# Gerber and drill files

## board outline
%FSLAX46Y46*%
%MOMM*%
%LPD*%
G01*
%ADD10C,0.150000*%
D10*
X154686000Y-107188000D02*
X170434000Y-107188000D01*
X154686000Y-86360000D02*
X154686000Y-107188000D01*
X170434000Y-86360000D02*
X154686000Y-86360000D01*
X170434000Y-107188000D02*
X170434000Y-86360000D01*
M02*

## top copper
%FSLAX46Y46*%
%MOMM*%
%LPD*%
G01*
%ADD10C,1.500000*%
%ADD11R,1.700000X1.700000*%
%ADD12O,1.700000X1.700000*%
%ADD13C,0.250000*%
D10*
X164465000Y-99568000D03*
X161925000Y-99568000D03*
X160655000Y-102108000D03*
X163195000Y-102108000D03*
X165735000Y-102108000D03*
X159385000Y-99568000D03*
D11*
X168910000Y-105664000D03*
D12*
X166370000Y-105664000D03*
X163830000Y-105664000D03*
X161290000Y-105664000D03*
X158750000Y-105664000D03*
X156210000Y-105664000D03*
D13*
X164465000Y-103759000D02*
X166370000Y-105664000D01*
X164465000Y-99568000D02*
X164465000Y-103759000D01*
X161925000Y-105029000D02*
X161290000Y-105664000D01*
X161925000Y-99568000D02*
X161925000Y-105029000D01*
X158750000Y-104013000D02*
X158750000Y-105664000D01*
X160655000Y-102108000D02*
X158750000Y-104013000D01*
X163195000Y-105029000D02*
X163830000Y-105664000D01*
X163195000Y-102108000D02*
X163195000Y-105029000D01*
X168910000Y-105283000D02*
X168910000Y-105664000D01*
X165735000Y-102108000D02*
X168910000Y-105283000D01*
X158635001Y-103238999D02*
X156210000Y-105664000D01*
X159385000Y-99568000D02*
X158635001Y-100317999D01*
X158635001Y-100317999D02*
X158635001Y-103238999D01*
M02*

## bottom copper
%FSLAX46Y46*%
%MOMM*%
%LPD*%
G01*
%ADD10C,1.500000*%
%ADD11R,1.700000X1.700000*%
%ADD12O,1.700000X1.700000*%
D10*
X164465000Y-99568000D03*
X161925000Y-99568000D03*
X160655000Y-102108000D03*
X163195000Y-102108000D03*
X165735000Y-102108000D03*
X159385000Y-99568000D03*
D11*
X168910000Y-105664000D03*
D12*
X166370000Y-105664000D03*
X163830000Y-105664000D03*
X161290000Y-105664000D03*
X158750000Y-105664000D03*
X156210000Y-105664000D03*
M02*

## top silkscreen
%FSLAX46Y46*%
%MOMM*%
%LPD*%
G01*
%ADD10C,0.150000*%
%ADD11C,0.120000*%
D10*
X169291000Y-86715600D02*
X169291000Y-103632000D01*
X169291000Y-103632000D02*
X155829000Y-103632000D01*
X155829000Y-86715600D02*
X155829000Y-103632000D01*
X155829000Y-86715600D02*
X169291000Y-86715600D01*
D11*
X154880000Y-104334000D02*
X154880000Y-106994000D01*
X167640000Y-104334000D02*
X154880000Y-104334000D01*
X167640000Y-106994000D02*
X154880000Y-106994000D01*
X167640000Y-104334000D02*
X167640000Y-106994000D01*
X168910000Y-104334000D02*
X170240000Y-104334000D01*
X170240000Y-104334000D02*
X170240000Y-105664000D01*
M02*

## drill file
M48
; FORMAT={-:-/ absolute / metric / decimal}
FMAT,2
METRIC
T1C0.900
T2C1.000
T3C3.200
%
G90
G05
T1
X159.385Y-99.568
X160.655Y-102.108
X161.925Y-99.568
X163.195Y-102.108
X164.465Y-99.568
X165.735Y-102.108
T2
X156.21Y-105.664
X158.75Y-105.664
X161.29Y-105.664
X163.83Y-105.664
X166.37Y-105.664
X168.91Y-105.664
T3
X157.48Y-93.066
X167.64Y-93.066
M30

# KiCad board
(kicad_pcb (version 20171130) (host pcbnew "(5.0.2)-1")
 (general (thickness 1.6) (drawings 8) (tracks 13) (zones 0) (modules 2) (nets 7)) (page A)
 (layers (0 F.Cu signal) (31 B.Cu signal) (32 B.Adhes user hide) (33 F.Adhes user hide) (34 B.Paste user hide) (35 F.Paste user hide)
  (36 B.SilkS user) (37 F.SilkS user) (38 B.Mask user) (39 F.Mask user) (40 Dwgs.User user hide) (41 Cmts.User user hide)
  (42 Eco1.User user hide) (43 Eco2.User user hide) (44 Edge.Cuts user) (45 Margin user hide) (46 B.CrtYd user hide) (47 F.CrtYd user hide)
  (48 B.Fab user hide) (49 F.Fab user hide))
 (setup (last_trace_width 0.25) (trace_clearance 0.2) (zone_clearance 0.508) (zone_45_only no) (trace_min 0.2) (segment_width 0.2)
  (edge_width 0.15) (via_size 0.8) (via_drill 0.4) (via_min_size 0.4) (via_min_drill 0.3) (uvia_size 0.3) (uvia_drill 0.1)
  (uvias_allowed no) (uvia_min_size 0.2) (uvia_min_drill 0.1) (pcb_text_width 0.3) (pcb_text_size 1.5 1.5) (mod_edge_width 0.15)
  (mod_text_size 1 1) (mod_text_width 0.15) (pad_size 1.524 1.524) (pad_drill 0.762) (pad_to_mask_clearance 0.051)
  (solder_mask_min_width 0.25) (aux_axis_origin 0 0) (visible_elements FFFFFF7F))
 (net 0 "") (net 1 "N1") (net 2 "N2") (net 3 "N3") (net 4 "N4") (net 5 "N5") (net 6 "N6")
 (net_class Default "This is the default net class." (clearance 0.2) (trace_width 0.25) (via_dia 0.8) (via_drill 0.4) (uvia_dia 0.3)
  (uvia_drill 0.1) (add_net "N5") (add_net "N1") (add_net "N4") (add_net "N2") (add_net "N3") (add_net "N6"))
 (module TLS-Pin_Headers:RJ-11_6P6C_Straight (layer F.Cu) (at 162.56 99.568 180)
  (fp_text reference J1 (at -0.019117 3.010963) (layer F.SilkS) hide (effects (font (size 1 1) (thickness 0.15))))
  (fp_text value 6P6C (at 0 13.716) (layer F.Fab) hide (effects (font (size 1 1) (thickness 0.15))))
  (fp_line (start -6.731 12.8524) (end -6.731 -4.064) (layer F.SilkS) (width 0.15))
  (fp_line (start -6.731 -4.064) (end 6.731 -4.064) (layer F.SilkS) (width 0.15))
  (fp_line (start 6.731 12.8524) (end 6.731 -4.064) (layer F.SilkS) (width 0.15))
  (fp_line (start 6.731 12.8524) (end -6.731 12.8524) (layer F.SilkS) (width 0.15))
  (pad "" np_thru_hole circle (at -5.08 6.5024) (size 3.2 3.2) (drill 3.2) (layers *.Cu *.Mask))
  (pad "" np_thru_hole circle (at 5.08 6.5024) (size 3.2 3.2) (drill 3.2) (layers *.Cu *.Mask))
  (pad 2 thru_hole circle (at -1.905 0) (size 1.5 1.5) (drill 0.9) (layers *.Cu *.Mask) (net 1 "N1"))
  (pad 4 thru_hole circle (at 0.635 0) (size 1.5 1.5) (drill 0.9) (layers *.Cu *.Mask) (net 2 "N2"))
  (pad 5 thru_hole circle (at 1.905 -2.54) (size 1.5 1.5) (drill 0.9) (layers *.Cu *.Mask) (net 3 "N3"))
  (pad 3 thru_hole circle (at -0.635 -2.54) (size 1.5 1.5) (drill 0.9) (layers *.Cu *.Mask) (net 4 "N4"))
  (pad 1 thru_hole circle (at -3.175 -2.54) (size 1.5 1.5) (drill 0.9) (layers *.Cu *.Mask) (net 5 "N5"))
  (pad 6 thru_hole circle (at 3.175 0) (size 1.5 1.5) (drill 0.9) (layers *.Cu *.Mask) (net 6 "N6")))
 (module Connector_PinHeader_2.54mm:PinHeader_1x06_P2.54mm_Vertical (layer F.Cu) (at 168.91 105.664 270)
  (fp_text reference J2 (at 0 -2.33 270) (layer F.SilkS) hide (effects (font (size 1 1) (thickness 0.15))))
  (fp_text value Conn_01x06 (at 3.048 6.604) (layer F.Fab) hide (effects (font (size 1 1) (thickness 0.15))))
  (fp_line (start -1.33 14.03) (end 1.33 14.03) (layer F.SilkS) (width 0.12))
  (fp_line (start -1.33 1.27) (end -1.33 14.03) (layer F.SilkS) (width 0.12))
  (fp_line (start 1.33 1.27) (end 1.33 14.03) (layer F.SilkS) (width 0.12))
  (fp_line (start -1.33 1.27) (end 1.33 1.27) (layer F.SilkS) (width 0.12))
  (fp_line (start -1.33 0) (end -1.33 -1.33) (layer F.SilkS) (width 0.12))
  (fp_line (start -1.33 -1.33) (end 0 -1.33) (layer F.SilkS) (width 0.12))
  (pad 1 thru_hole rect (at 0 0 270) (size 1.7 1.7) (drill 1) (layers *.Cu *.Mask) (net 5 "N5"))
  (pad 2 thru_hole oval (at 0 2.54 270) (size 1.7 1.7) (drill 1) (layers *.Cu *.Mask) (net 1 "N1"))
  (pad 3 thru_hole oval (at 0 5.08 270) (size 1.7 1.7) (drill 1) (layers *.Cu *.Mask) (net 4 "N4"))
  (pad 4 thru_hole oval (at 0 7.62 270) (size 1.7 1.7) (drill 1) (layers *.Cu *.Mask) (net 2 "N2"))
  (pad 5 thru_hole oval (at 0 10.16 270) (size 1.7 1.7) (drill 1) (layers *.Cu *.Mask) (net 3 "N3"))
  (pad 6 thru_hole oval (at 0 12.7 270) (size 1.7 1.7) (drill 1) (layers *.Cu *.Mask) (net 6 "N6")))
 (gr_line (start 154.686 107.188) (end 170.434 107.188) (layer Edge.Cuts) (width 0.15))
 (gr_line (start 154.686 86.36) (end 154.686 107.188) (layer Edge.Cuts) (width 0.15))
 (gr_line (start 170.434 86.36) (end 154.686 86.36) (layer Edge.Cuts) (width 0.15))
 (gr_line (start 170.434 107.188) (end 170.434 86.36) (layer Edge.Cuts) (width 0.15))
 (segment (start 164.465 103.759) (end 166.37 105.664) (width 0.25) (layer F.Cu) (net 1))
 (segment (start 164.465 99.568) (end 164.465 103.759) (width 0.25) (layer F.Cu) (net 1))
 (segment (start 161.925 105.029) (end 161.29 105.664) (width 0.25) (layer F.Cu) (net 2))
 (segment (start 161.925 99.568) (end 161.925 105.029) (width 0.25) (layer F.Cu) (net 2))
 (segment (start 158.75 104.013) (end 158.75 105.664) (width 0.25) (layer F.Cu) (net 3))
 (segment (start 160.655 102.108) (end 158.75 104.013) (width 0.25) (layer F.Cu) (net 3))
 (segment (start 163.195 105.029) (end 163.83 105.664) (width 0.25) (layer F.Cu) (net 4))
 (segment (start 163.195 102.108) (end 163.195 105.029) (width 0.25) (layer F.Cu) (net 4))
 (segment (start 168.91 105.283) (end 168.91 105.664) (width 0.25) (layer F.Cu) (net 5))
 (segment (start 165.735 102.108) (end 168.91 105.283) (width 0.25) (layer F.Cu) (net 5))
 (segment (start 158.635001 103.238999) (end 156.21 105.664) (width 0.25) (layer F.Cu) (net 6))
 (segment (start 159.385 99.568) (end 158.635001 100.317999) (width 0.25) (layer F.Cu) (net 6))
 (segment (start 158.635001 100.317999) (end 158.635001 103.238999) (width 0.25) (layer F.Cu) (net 6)))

